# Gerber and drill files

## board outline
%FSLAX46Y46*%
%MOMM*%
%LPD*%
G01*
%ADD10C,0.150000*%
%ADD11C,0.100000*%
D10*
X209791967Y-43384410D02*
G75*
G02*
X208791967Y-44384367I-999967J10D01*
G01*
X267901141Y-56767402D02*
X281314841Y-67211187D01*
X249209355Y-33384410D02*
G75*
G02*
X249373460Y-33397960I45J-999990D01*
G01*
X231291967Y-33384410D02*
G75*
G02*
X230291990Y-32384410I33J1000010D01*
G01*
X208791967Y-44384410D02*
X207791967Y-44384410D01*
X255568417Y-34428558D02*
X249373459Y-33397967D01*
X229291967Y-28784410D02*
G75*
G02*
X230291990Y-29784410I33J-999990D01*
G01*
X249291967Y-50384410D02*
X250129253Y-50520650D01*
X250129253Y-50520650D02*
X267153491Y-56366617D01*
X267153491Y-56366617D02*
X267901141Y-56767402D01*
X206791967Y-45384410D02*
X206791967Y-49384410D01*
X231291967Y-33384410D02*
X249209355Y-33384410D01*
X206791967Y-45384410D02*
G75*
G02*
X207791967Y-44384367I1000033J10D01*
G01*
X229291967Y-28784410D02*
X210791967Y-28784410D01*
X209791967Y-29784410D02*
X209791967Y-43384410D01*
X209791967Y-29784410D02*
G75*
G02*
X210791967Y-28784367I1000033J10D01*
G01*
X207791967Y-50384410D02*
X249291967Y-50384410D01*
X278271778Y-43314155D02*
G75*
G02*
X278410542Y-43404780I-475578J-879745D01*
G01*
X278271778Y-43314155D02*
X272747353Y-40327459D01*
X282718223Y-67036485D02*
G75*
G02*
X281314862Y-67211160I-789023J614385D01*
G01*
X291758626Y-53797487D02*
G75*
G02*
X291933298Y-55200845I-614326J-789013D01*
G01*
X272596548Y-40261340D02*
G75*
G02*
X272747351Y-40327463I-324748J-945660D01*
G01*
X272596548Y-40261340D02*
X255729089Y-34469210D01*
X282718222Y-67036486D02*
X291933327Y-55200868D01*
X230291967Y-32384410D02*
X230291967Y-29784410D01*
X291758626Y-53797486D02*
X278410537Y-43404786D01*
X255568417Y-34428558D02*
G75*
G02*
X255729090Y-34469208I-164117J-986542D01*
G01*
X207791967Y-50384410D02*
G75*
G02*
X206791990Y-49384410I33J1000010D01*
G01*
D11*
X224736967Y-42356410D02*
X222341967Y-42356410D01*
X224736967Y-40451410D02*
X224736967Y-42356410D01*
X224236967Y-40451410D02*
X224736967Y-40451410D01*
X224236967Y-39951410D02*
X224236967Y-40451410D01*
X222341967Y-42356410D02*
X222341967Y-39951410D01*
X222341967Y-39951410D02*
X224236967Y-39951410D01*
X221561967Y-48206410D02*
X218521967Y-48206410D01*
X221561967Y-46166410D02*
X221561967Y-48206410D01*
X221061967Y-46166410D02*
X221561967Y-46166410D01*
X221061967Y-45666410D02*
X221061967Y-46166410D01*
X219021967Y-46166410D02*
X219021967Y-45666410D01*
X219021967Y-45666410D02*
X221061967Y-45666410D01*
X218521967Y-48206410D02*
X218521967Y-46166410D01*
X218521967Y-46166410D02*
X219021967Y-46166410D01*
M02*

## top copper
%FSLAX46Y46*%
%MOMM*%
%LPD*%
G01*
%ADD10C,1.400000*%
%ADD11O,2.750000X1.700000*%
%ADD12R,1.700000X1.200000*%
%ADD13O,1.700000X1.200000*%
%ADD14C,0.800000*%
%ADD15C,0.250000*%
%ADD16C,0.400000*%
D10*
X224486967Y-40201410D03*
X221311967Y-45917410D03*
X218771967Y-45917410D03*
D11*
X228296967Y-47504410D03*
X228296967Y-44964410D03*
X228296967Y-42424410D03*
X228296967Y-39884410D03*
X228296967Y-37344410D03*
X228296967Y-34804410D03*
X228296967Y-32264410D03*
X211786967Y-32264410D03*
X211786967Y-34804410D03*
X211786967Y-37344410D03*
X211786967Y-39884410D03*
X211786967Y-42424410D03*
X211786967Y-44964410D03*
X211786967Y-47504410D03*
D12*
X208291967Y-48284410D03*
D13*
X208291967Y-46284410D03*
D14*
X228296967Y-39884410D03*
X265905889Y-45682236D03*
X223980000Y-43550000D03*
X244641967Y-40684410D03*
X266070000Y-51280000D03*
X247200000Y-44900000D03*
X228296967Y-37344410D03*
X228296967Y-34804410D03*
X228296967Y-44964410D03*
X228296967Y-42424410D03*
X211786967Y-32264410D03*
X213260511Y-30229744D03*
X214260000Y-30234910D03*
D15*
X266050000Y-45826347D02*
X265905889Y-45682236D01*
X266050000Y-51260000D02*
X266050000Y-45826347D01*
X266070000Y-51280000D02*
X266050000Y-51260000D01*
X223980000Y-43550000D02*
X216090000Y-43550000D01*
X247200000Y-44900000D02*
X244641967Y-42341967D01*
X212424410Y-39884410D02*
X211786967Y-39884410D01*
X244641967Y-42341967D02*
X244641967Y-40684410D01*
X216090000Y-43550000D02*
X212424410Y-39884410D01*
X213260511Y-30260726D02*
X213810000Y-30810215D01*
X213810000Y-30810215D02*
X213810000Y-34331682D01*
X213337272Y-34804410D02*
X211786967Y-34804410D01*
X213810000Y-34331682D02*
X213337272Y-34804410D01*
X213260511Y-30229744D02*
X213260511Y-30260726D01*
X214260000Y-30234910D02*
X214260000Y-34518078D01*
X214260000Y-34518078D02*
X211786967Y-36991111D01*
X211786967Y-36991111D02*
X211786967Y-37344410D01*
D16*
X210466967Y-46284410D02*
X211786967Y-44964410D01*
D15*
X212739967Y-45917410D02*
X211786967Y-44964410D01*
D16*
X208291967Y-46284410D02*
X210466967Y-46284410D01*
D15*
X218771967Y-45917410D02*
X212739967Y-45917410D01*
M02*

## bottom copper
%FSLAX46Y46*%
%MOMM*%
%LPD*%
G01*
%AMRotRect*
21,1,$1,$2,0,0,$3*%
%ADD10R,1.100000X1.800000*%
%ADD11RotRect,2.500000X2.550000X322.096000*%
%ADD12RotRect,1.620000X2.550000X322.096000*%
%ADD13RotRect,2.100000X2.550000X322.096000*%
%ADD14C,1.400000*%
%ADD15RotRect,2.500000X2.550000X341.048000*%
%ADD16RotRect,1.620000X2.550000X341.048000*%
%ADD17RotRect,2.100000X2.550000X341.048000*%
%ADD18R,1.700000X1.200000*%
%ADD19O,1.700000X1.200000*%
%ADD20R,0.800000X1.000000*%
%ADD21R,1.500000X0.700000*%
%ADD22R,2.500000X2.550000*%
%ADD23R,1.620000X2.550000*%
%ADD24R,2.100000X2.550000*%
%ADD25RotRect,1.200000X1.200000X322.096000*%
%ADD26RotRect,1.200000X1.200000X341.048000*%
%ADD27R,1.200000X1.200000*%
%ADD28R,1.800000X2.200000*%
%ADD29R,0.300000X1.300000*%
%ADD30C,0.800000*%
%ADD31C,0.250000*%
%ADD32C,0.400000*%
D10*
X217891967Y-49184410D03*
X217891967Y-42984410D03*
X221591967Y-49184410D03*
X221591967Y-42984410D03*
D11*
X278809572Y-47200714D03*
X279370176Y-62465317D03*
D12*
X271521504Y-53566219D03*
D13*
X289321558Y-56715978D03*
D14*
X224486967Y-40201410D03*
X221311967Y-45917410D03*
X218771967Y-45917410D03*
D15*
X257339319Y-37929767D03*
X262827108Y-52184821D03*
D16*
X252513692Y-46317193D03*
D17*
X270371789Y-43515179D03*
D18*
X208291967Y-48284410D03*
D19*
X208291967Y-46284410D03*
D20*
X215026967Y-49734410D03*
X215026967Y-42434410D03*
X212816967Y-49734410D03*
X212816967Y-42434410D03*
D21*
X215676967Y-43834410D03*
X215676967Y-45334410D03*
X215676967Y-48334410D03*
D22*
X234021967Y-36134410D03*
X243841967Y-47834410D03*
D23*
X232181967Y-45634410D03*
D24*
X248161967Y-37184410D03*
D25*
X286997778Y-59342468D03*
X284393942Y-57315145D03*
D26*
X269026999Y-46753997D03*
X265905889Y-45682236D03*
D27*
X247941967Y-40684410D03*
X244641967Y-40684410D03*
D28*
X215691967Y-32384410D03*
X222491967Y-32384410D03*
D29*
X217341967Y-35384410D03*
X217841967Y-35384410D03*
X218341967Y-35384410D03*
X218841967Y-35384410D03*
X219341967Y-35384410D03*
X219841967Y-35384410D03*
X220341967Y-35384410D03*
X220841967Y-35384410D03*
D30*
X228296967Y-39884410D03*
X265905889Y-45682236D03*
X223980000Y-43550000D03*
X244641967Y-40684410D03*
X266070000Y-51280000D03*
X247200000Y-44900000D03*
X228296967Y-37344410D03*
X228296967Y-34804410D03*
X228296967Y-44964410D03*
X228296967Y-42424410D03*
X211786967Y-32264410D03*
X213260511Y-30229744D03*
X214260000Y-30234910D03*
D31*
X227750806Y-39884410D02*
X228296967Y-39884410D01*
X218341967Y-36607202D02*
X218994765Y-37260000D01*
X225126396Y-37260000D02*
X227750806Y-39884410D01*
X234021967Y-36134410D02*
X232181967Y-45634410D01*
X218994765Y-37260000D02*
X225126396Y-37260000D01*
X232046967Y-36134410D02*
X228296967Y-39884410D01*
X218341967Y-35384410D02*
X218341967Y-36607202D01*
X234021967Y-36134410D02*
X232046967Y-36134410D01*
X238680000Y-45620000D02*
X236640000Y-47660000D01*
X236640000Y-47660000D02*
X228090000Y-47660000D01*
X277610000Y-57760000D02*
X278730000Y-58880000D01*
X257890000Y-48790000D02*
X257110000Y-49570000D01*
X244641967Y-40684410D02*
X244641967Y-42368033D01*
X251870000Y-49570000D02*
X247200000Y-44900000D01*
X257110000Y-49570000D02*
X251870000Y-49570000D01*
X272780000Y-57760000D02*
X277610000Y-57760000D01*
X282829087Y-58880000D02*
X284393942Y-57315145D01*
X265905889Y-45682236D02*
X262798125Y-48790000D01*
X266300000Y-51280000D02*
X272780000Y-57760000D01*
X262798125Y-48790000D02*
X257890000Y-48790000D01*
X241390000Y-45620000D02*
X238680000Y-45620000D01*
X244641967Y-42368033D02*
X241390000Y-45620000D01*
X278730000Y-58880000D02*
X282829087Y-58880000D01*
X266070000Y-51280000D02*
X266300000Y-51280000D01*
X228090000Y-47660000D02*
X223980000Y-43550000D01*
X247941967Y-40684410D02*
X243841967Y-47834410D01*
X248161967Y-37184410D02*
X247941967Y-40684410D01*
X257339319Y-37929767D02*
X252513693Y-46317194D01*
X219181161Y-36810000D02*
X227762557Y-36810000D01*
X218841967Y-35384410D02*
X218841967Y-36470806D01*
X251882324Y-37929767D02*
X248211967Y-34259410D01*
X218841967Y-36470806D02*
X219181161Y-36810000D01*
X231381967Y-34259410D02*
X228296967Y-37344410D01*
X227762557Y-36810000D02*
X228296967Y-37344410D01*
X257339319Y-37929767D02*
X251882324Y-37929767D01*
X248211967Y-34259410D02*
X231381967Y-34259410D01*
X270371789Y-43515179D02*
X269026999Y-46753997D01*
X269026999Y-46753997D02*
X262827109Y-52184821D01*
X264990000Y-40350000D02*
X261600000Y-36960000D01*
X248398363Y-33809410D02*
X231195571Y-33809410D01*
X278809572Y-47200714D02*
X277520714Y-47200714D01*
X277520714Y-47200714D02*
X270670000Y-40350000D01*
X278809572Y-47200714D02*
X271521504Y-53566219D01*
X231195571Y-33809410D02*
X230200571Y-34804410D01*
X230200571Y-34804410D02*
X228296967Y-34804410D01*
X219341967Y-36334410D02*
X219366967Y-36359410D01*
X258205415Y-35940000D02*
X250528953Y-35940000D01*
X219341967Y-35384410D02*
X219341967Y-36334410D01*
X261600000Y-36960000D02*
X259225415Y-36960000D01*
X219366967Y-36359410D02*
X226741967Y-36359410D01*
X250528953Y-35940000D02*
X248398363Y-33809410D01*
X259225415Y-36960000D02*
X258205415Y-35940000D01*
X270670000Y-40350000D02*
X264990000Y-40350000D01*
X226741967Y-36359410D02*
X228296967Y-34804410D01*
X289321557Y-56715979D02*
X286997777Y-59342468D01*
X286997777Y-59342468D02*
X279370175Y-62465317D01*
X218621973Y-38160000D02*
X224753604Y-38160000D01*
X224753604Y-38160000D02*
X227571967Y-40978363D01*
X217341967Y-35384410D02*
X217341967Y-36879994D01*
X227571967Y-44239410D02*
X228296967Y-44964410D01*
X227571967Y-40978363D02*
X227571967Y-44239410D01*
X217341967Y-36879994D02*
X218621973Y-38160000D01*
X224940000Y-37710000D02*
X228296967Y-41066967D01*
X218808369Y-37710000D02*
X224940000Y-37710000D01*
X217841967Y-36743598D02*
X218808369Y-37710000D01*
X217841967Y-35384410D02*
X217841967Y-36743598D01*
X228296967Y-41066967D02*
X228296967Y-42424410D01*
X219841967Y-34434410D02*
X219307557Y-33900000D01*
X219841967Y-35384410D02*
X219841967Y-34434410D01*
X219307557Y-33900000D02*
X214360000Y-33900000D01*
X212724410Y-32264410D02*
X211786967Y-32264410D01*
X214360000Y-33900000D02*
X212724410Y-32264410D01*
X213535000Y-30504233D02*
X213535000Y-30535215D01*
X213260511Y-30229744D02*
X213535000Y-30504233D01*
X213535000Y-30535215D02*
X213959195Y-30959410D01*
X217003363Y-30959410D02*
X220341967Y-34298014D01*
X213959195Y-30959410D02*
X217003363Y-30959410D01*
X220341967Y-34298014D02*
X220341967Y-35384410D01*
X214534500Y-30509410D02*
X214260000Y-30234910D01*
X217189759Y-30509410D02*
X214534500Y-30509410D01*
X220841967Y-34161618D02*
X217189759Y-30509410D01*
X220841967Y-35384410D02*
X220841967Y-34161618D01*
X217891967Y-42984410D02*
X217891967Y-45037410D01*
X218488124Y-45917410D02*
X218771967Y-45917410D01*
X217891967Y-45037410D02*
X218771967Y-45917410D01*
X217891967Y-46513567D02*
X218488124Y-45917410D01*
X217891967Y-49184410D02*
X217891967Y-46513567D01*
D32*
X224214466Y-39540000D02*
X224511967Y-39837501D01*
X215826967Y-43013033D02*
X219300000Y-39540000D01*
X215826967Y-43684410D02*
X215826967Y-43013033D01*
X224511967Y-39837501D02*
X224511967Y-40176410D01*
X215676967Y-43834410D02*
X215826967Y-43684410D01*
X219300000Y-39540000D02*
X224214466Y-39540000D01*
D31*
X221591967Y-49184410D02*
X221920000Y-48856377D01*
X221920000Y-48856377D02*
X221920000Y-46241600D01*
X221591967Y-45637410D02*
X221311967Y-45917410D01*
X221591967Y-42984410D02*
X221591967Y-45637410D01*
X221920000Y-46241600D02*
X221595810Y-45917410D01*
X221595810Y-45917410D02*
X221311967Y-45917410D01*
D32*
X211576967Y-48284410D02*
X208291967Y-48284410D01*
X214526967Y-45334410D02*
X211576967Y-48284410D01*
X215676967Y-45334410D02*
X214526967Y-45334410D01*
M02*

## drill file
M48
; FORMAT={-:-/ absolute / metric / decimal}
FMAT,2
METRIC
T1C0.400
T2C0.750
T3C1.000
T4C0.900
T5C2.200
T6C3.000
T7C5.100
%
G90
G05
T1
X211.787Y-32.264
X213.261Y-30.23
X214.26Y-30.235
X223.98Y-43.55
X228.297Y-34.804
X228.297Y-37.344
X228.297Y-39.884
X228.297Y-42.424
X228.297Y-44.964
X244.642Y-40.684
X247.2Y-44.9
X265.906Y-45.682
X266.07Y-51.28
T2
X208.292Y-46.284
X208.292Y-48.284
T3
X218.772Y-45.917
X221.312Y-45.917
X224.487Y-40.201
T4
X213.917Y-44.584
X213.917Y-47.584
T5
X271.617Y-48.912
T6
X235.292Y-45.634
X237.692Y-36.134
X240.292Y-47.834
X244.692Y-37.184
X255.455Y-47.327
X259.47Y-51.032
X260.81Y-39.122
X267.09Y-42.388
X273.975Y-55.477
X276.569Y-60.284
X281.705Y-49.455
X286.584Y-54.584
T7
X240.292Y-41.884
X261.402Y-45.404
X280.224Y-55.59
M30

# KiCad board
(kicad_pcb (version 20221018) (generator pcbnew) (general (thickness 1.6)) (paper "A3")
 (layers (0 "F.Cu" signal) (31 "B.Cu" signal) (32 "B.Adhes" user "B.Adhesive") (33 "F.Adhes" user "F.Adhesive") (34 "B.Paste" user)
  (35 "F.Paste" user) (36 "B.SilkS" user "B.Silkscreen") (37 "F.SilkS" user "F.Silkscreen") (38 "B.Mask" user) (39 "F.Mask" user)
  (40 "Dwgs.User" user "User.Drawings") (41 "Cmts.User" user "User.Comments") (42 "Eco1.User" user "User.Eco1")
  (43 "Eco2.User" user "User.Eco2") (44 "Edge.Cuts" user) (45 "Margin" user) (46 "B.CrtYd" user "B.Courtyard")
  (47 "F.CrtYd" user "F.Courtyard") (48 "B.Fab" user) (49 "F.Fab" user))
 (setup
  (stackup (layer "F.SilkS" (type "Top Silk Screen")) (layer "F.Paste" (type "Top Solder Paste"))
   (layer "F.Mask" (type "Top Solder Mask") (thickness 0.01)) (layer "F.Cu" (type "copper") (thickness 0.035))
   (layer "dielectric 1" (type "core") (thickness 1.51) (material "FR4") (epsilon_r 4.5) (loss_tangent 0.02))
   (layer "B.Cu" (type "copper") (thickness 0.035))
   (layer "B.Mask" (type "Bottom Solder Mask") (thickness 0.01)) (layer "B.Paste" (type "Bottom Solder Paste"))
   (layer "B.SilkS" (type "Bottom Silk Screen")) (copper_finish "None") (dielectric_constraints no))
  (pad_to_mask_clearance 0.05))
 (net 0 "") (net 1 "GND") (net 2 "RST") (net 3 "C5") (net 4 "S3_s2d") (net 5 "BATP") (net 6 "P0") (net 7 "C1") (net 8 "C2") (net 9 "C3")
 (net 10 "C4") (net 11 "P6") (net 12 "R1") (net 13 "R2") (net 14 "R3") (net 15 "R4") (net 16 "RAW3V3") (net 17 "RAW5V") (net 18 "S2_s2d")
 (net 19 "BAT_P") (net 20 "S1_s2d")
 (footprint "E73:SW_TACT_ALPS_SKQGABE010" (layer "F.Cu") (at 219.741967 46.08441 90)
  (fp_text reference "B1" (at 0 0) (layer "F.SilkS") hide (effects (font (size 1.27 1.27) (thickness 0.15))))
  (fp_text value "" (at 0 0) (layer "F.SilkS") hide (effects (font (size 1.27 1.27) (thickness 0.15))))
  (pad "1" smd rect (at -3.1 -1.85 90) (size 1.8 1.1) (layers "B.Cu" "B.Paste" "B.Mask") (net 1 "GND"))
  (pad "1" smd rect (at 3.1 -1.85 90) (size 1.8 1.1) (layers "B.Cu" "B.Paste" "B.Mask") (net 1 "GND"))
  (pad "2" smd rect (at -3.1 1.85 90) (size 1.8 1.1) (layers "B.Cu" "B.Paste" "B.Mask") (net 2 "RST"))
  (pad "2" smd rect (at 3.1 1.85 90) (size 1.8 1.1) (layers "B.Cu" "B.Paste" "B.Mask") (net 2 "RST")))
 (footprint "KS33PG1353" (layer "F.Cu") (at 280.224404 55.589614 -37.904)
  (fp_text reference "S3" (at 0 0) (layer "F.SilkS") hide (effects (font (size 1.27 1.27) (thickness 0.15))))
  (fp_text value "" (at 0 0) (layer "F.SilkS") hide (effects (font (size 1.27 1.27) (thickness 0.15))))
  (pad "" np_thru_hole circle (at -5 3.75) (size 3 3) (drill 3) (layers "*.Cu" "*.Mask"))
  (pad "" np_thru_hole circle (at -2.6 -5.75) (size 3 3) (drill 3) (layers "*.Cu" "*.Mask"))
  (pad "" np_thru_hole circle (at 0 0) (size 5.1 5.1) (drill 5.1) (layers "*.Cu" "*.Mask"))
  (pad "" np_thru_hole circle (at 0 5.95) (size 3 3) (drill 3) (layers "*.Cu" "*.Mask"))
  (pad "" np_thru_hole circle (at 4.4 -4.7) (size 3 3) (drill 3) (layers "*.Cu" "*.Mask"))
  (pad "1" smd rect (at -6.27 -5.75 322.096) (size 2.5 2.55) (layers "B.Cu" "B.Paste" "B.Mask") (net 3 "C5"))
  (pad "1" smd rect (at 3.55 5.95 322.096) (size 2.5 2.55) (layers "B.Cu" "B.Paste" "B.Mask") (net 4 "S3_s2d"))
  (pad "2" smd rect (at -8.11 3.75 322.096) (size 1.62 2.55) (layers "B.Cu" "B.Paste" "B.Mask") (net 3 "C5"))
  (pad "2" smd rect (at 7.87 -4.7 322.096) (size 2.1 2.55) (layers "B.Cu" "B.Paste" "B.Mask") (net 4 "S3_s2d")))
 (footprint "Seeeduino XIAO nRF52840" (layer "F.Cu") (at 220.041967 39.88441 180)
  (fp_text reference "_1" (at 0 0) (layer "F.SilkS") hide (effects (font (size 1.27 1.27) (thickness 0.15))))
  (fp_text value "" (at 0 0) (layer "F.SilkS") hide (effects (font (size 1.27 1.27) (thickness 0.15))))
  (fp_line (start -4.695 -2.472) (end -2.3 -2.472) (stroke (width 0.1) (type solid)) (layer "Edge.Cuts"))
  (fp_line (start -4.695 -0.567) (end -4.695 -2.472) (stroke (width 0.1) (type solid)) (layer "Edge.Cuts"))
  (fp_line (start -4.195 -0.567) (end -4.695 -0.567) (stroke (width 0.1) (type solid)) (layer "Edge.Cuts"))
  (fp_line (start -4.195 -0.067) (end -4.195 -0.567) (stroke (width 0.1) (type solid)) (layer "Edge.Cuts"))
  (fp_line (start -2.3 -2.472) (end -2.3 -0.067) (stroke (width 0.1) (type solid)) (layer "Edge.Cuts"))
  (fp_line (start -2.3 -0.067) (end -4.195 -0.067) (stroke (width 0.1) (type solid)) (layer "Edge.Cuts"))
  (fp_line (start -1.52 -8.322) (end 1.52 -8.322) (stroke (width 0.1) (type solid)) (layer "Edge.Cuts"))
  (fp_line (start -1.52 -6.282) (end -1.52 -8.322) (stroke (width 0.1) (type solid)) (layer "Edge.Cuts"))
  (fp_line (start -1.02 -6.282) (end -1.52 -6.282) (stroke (width 0.1) (type solid)) (layer "Edge.Cuts"))
  (fp_line (start -1.02 -5.782) (end -1.02 -6.282) (stroke (width 0.1) (type solid)) (layer "Edge.Cuts"))
  (fp_line (start 1.02 -6.282) (end 1.02 -5.782) (stroke (width 0.1) (type solid)) (layer "Edge.Cuts"))
  (fp_line (start 1.02 -5.782) (end -1.02 -5.782) (stroke (width 0.1) (type solid)) (layer "Edge.Cuts"))
  (fp_line (start 1.52 -8.322) (end 1.52 -6.282) (stroke (width 0.1) (type solid)) (layer "Edge.Cuts"))
  (fp_line (start 1.52 -6.282) (end 1.02 -6.282) (stroke (width 0.1) (type solid)) (layer "Edge.Cuts"))
  (pad "" thru_hole circle (at -4.445 -0.317) (size 1.4 1.4) (drill 1) (layers "*.Cu" "*.Mask") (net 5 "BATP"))
  (pad "" thru_hole circle (at -1.27 -6.033) (size 1.4 1.4) (drill 1) (layers "*.Cu" "*.Mask") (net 2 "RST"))
  (pad "" thru_hole circle (at 1.27 -6.033) (size 1.4 1.4) (drill 1) (layers "*.Cu" "*.Mask") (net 1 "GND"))
  (pad "1" smd oval (at -8.255 -7.62 180) (size 2.75 1.7) (layers "F.Cu" "F.Paste" "F.Mask") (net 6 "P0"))
  (pad "2" smd oval (at -8.255 -5.08 180) (size 2.75 1.7) (layers "F.Cu" "F.Paste" "F.Mask") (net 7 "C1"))
  (pad "3" smd oval (at -8.255 -2.54 180) (size 2.75 1.7) (layers "F.Cu" "F.Paste" "F.Mask") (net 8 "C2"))
  (pad "4" smd oval (at -8.255 0 180) (size 2.75 1.7) (layers "F.Cu" "F.Paste" "F.Mask") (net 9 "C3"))
  (pad "5" smd oval (at -8.255 2.54 180) (size 2.75 1.7) (layers "F.Cu" "F.Paste" "F.Mask") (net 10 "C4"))
  (pad "6" smd oval (at -8.255 5.08 180) (size 2.75 1.7) (layers "F.Cu" "F.Paste" "F.Mask") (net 3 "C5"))
  (pad "7" smd oval (at -8.255 7.62 180) (size 2.75 1.7) (layers "F.Cu" "F.Paste" "F.Mask") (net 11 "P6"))
  (pad "8" smd oval (at 8.255 7.62 180) (size 2.75 1.7) (layers "F.Cu" "F.Paste" "F.Mask") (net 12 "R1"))
  (pad "9" smd oval (at 8.255 5.08 180) (size 2.75 1.7) (layers "F.Cu" "F.Paste" "F.Mask") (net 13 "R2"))
  (pad "10" smd oval (at 8.255 2.54 180) (size 2.75 1.7) (layers "F.Cu" "F.Paste" "F.Mask") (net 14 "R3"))
  (pad "11" smd oval (at 8.255 0 180) (size 2.75 1.7) (layers "F.Cu" "F.Paste" "F.Mask") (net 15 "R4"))
  (pad "12" smd oval (at 8.255 -2.54 180) (size 2.75 1.7) (layers "F.Cu" "F.Paste" "F.Mask") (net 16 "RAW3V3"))
  (pad "13" smd oval (at 8.255 -5.08 180) (size 2.75 1.7) (layers "F.Cu" "F.Paste" "F.Mask") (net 1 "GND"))
  (pad "14" smd oval (at 8.255 -7.62 180) (size 2.75 1.7) (layers "F.Cu" "F.Paste" "F.Mask") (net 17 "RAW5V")))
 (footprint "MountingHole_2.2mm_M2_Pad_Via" (layer "F.Cu") (at 271.61651 48.91199 -18.952)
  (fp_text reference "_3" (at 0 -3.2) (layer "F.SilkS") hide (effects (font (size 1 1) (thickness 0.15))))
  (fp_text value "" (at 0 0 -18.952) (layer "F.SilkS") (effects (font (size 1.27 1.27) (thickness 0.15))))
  (pad "" np_thru_hole circle (at 0 0) (size 2.2 2.2) (drill 2.2) (layers "*.Cu" "*.Mask")))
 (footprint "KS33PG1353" (layer "F.Cu") (at 261.401967 45.40441 -18.952)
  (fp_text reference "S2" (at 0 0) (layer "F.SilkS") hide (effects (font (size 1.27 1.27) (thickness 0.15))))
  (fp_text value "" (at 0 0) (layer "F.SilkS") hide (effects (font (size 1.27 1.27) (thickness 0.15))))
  (pad "" np_thru_hole circle (at -5 3.75) (size 3 3) (drill 3) (layers "*.Cu" "*.Mask"))
  (pad "" np_thru_hole circle (at -2.6 -5.75) (size 3 3) (drill 3) (layers "*.Cu" "*.Mask"))
  (pad "" np_thru_hole circle (at 0 0) (size 5.1 5.1) (drill 5.1) (layers "*.Cu" "*.Mask"))
  (pad "" np_thru_hole circle (at 0 5.95) (size 3 3) (drill 3) (layers "*.Cu" "*.Mask"))
  (pad "" np_thru_hole circle (at 4.4 -4.7) (size 3 3) (drill 3) (layers "*.Cu" "*.Mask"))
  (pad "1" smd rect (at -6.27 -5.75 341.048) (size 2.5 2.55) (layers "B.Cu" "B.Paste" "B.Mask") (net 10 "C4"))
  (pad "1" smd rect (at 3.55 5.95 341.048) (size 2.5 2.55) (layers "B.Cu" "B.Paste" "B.Mask") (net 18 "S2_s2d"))
  (pad "2" smd rect (at -8.11 3.75 341.048) (size 1.62 2.55) (layers "B.Cu" "B.Paste" "B.Mask") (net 10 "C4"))
  (pad "2" smd rect (at 7.87 -4.7 341.048) (size 2.1 2.55) (layers "B.Cu" "B.Paste" "B.Mask") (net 18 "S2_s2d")))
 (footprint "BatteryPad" (layer "F.Cu") (at 208.291967 47.28441 90)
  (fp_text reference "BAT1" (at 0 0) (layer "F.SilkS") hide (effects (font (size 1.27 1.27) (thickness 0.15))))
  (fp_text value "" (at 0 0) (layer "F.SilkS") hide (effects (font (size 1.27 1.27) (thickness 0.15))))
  (pad "1" thru_hole rect (at -1 0 90) (size 1.2 1.7) (drill 0.75) (layers "*.Cu" "*.Mask") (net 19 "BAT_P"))
  (pad "2" thru_hole oval (at 1 0 90) (size 1.2 1.7) (drill 0.75) (layers "*.Cu" "*.Mask") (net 1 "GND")))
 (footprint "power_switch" (layer "F.Cu") (at 213.941967 46.08441 180)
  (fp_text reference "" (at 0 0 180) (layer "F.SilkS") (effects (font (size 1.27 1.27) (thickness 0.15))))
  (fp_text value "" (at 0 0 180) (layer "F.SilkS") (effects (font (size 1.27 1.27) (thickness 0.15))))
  (pad "" smd rect (at -1.085 -3.65 90) (size 1 0.8) (layers "B.Cu" "B.Paste" "B.Mask"))
  (pad "" smd rect (at -1.085 3.65 90) (size 1 0.8) (layers "B.Cu" "B.Paste" "B.Mask"))
  (pad "" np_thru_hole circle (at 0.025 -1.5 270) (size 0.9 0.9) (drill 0.9) (layers "*.Cu" "*.Mask"))
  (pad "" np_thru_hole circle (at 0.025 1.5 270) (size 0.9 0.9) (drill 0.9) (layers "*.Cu" "*.Mask"))
  (pad "" smd rect (at 1.125 -3.65 90) (size 1 0.8) (layers "B.Cu" "B.Paste" "B.Mask"))
  (pad "" smd rect (at 1.125 3.65 90) (size 1 0.8) (layers "B.Cu" "B.Paste" "B.Mask"))
  (pad "4" smd rect (at -1.735 2.25 90) (size 0.7 1.5) (layers "B.Cu" "B.Paste" "B.Mask") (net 5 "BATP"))
  (pad "5" smd rect (at -1.735 0.75 90) (size 0.7 1.5) (layers "B.Cu" "B.Paste" "B.Mask") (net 19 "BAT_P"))
  (pad "6" smd rect (at -1.735 -2.25 90) (size 0.7 1.5) (layers "B.Cu" "B.Paste" "B.Mask")))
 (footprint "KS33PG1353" (layer "F.Cu") (at 240.291967 41.88441)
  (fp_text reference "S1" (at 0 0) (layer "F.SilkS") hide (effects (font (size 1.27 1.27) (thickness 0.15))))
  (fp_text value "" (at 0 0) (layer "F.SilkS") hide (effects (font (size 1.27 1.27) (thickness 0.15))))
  (pad "" np_thru_hole circle (at -5 3.75) (size 3 3) (drill 3) (layers "*.Cu" "*.Mask"))
  (pad "" np_thru_hole circle (at -2.6 -5.75) (size 3 3) (drill 3) (layers "*.Cu" "*.Mask"))
  (pad "" np_thru_hole circle (at 0 0) (size 5.1 5.1) (drill 5.1) (layers "*.Cu" "*.Mask"))
  (pad "" np_thru_hole circle (at 0 5.95) (size 3 3) (drill 3) (layers "*.Cu" "*.Mask"))
  (pad "" np_thru_hole circle (at 4.4 -4.7) (size 3 3) (drill 3) (layers "*.Cu" "*.Mask"))
  (pad "1" smd rect (at -6.27 -5.75) (size 2.5 2.55) (layers "B.Cu" "B.Paste" "B.Mask") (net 9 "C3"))
  (pad "1" smd rect (at 3.55 5.95) (size 2.5 2.55) (layers "B.Cu" "B.Paste" "B.Mask") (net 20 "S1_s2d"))
  (pad "2" smd rect (at -8.11 3.75) (size 1.62 2.55) (layers "B.Cu" "B.Paste" "B.Mask") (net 9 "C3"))
  (pad "2" smd rect (at 7.87 -4.7) (size 2.1 2.55) (layers "B.Cu" "B.Paste" "B.Mask") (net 20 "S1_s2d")))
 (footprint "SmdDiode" (layer "B.Cu") (at 280.224404 55.589614 -37.904)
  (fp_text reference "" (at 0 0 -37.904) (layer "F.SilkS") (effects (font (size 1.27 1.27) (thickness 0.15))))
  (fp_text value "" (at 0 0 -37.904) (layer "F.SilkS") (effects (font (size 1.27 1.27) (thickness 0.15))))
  (pad "1" smd rect (at 7.65 -1.2 322.096) (size 1.2 1.2) (layers "B.Cu" "B.Paste" "B.Mask") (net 4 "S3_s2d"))
  (pad "2" smd rect (at 4.35 -1.2 322.096) (size 1.2 1.2) (layers "B.Cu" "B.Paste" "B.Mask") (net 15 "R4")))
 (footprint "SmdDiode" (layer "B.Cu") (at 261.401967 45.40441 -18.952)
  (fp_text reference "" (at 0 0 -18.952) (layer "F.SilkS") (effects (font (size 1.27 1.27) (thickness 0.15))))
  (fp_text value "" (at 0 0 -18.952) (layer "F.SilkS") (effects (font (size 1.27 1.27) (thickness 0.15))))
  (pad "1" smd rect (at 7.65 -1.2 341.048) (size 1.2 1.2) (layers "B.Cu" "B.Paste" "B.Mask") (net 18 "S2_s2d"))
  (pad "2" smd rect (at 4.35 -1.2 341.048) (size 1.2 1.2) (layers "B.Cu" "B.Paste" "B.Mask") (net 15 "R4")))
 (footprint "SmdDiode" (layer "B.Cu") (at 240.291967 41.88441)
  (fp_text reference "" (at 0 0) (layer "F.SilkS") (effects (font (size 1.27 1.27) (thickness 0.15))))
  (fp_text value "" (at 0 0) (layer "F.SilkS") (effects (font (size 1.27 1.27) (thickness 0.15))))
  (pad "1" smd rect (at 7.65 -1.2) (size 1.2 1.2) (layers "B.Cu" "B.Paste" "B.Mask") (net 20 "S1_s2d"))
  (pad "2" smd rect (at 4.35 -1.2) (size 1.2 1.2) (layers "B.Cu" "B.Paste" "B.Mask") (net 15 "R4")))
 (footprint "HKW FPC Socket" (layer "B.Cu") (at 219.091967 32.38441)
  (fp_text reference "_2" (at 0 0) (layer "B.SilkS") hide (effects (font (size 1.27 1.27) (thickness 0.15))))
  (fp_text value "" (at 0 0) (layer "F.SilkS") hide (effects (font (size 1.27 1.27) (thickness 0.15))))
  (pad "" smd rect (at -3.4 0) (size 1.8 2.2) (layers "B.Cu" "B.Paste" "B.Mask"))
  (pad "" smd rect (at 3.4 0) (size 1.8 2.2) (layers "B.Cu" "B.Paste" "B.Mask"))
  (pad "1" smd rect (at -1.75 3) (size 0.3 1.3) (layers "B.Cu" "B.Paste" "B.Mask") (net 7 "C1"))
  (pad "2" smd rect (at -1.25 3) (size 0.3 1.3) (layers "B.Cu" "B.Paste" "B.Mask") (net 8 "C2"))
  (pad "3" smd rect (at -0.75 3) (size 0.3 1.3) (layers "B.Cu" "B.Paste" "B.Mask") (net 9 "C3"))
  (pad "4" smd rect (at -0.25 3) (size 0.3 1.3) (layers "B.Cu" "B.Paste" "B.Mask") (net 10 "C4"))
  (pad "5" smd rect (at 0.25 3) (size 0.3 1.3) (layers "B.Cu" "B.Paste" "B.Mask") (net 3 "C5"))
  (pad "6" smd rect (at 0.75 3) (size 0.3 1.3) (layers "B.Cu" "B.Paste" "B.Mask") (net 12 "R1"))
  (pad "7" smd rect (at 1.25 3) (size 0.3 1.3) (layers "B.Cu" "B.Paste" "B.Mask") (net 13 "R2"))
  (pad "8" smd rect (at 1.75 3) (size 0.3 1.3) (layers "B.Cu" "B.Paste" "B.Mask") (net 14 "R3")))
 (gr_arc (start 209.791967 43.38441) (mid 209.499074 44.091517) (end 208.791967 44.38441) (stroke (width 0.15) (type solid))
  (layer "Edge.Cuts"))
 (gr_line (start 267.901141 56.767402) (end 281.314841 67.211187) (stroke (width 0.15) (type solid)) (layer "Edge.Cuts"))
 (gr_arc (start 249.209355 33.38441) (mid 249.291687 33.387805) (end 249.373459 33.397967) (stroke (width 0.15) (type solid))
  (layer "Edge.Cuts"))
 (gr_arc (start 231.291967 33.38441) (mid 230.58486 33.091517) (end 230.291967 32.38441) (stroke (width 0.15) (type solid))
  (layer "Edge.Cuts"))
 (gr_line (start 208.791967 44.38441) (end 207.791967 44.38441) (stroke (width 0.15) (type solid)) (layer "Edge.Cuts"))
 (gr_line (start 255.568417 34.428558) (end 249.373459 33.397967) (stroke (width 0.15) (type solid)) (layer "Edge.Cuts"))
 (gr_arc (start 229.291967 28.78441) (mid 229.999074 29.077303) (end 230.291967 29.78441) (stroke (width 0.15) (type solid))
  (layer "Edge.Cuts"))
 (gr_line (start 249.291967 50.38441) (end 250.129253 50.52065) (stroke (width 0.15) (type solid)) (layer "Edge.Cuts"))
 (gr_line (start 250.129253 50.52065) (end 267.153491 56.366617) (stroke (width 0.15) (type solid)) (layer "Edge.Cuts"))
 (gr_line (start 267.153491 56.366617) (end 267.901141 56.767402) (stroke (width 0.15) (type solid)) (layer "Edge.Cuts"))
 (gr_line (start 206.791967 45.38441) (end 206.791967 49.38441) (stroke (width 0.15) (type solid)) (layer "Edge.Cuts"))
 (gr_line (start 231.291967 33.38441) (end 249.209355 33.38441) (stroke (width 0.15) (type solid)) (layer "Edge.Cuts"))
 (gr_arc (start 206.791967 45.38441) (mid 207.08486 44.677303) (end 207.791967 44.38441) (stroke (width 0.15) (type solid))
  (layer "Edge.Cuts"))
 (gr_line (start 229.291967 28.78441) (end 210.791967 28.78441) (stroke (width 0.15) (type solid)) (layer "Edge.Cuts"))
 (gr_line (start 209.791967 29.78441) (end 209.791967 43.38441) (stroke (width 0.15) (type solid)) (layer "Edge.Cuts"))
 (gr_arc (start 209.791967 29.78441) (mid 210.08486 29.077303) (end 210.791967 28.78441) (stroke (width 0.15) (type solid))
  (layer "Edge.Cuts"))
 (gr_line (start 207.791967 50.38441) (end 249.291967 50.38441) (stroke (width 0.15) (type solid)) (layer "Edge.Cuts"))
 (gr_arc (start 278.271778 43.314155) (mid 278.343038 43.356591) (end 278.410537 43.404786) (stroke (width 0.15) (type solid))
  (layer "Edge.Cuts"))
 (gr_line (start 278.271778 43.314155) (end 272.747353 40.327459) (stroke (width 0.15) (type solid)) (layer "Edge.Cuts"))
 (gr_arc (start 282.718223 67.036485) (mid 282.052714 67.414486) (end 281.314841 67.211187) (stroke (width 0.15) (type solid))
  (layer "Edge.Cuts"))
 (gr_arc (start 291.758626 53.797487) (mid 292.136626 54.462996) (end 291.933327 55.200868) (stroke (width 0.15) (type solid))
  (layer "Edge.Cuts"))
 (gr_arc (start 272.596548 40.26134) (mid 272.673314 40.29129) (end 272.747353 40.327459) (stroke (width 0.15) (type solid))
  (layer "Edge.Cuts"))
 (gr_line (start 272.596548 40.26134) (end 255.729089 34.46921) (stroke (width 0.15) (type solid)) (layer "Edge.Cuts"))
 (gr_line (start 282.718222 67.036486) (end 291.933327 55.200868) (stroke (width 0.15) (type solid)) (layer "Edge.Cuts"))
 (gr_line (start 230.291967 32.38441) (end 230.291967 29.78441) (stroke (width 0.15) (type solid)) (layer "Edge.Cuts"))
 (gr_line (start 291.758626 53.797486) (end 278.410537 43.404786) (stroke (width 0.15) (type solid)) (layer "Edge.Cuts"))
 (gr_arc (start 255.568417 34.428558) (mid 255.649597 34.44555) (end 255.729089 34.46921) (stroke (width 0.15) (type solid))
  (layer "Edge.Cuts"))
 (gr_arc (start 207.791967 50.38441) (mid 207.08486 50.091517) (end 206.791967 49.38441) (stroke (width 0.15) (type solid))
  (layer "Edge.Cuts"))
 (via (at 228.296967 39.88441) (size 0.8) (drill 0.4) (layers "F.Cu" "B.Cu") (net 9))
 (segment (start 227.750806 39.88441) (end 228.296967 39.88441) (width 0.25) (layer "B.Cu") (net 9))
 (segment (start 218.341967 36.607202) (end 218.994765 37.26) (width 0.25) (layer "B.Cu") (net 9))
 (segment (start 225.126396 37.26) (end 227.750806 39.88441) (width 0.25) (layer "B.Cu") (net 9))
 (segment (start 234.021967 36.13441) (end 232.181967 45.63441) (width 0.25) (layer "B.Cu") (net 9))
 (segment (start 218.994765 37.26) (end 225.126396 37.26) (width 0.25) (layer "B.Cu") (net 9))
 (segment (start 232.046967 36.13441) (end 228.296967 39.88441) (width 0.25) (layer "B.Cu") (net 9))
 (segment (start 218.341967 35.38441) (end 218.341967 36.607202) (width 0.25) (layer "B.Cu") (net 9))
 (segment (start 234.021967 36.13441) (end 232.046967 36.13441) (width 0.25) (layer "B.Cu") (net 9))
 (segment (start 266.05 45.826347) (end 265.905889 45.682236) (width 0.25) (layer "F.Cu") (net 15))
 (segment (start 266.05 51.26) (end 266.05 45.826347) (width 0.25) (layer "F.Cu") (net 15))
 (segment (start 266.07 51.28) (end 266.05 51.26) (width 0.25) (layer "F.Cu") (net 15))
 (segment (start 223.98 43.55) (end 216.09 43.55) (width 0.25) (layer "F.Cu") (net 15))
 (segment (start 247.2 44.9) (end 244.641967 42.341967) (width 0.25) (layer "F.Cu") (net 15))
 (segment (start 212.42441 39.88441) (end 211.786967 39.88441) (width 0.25) (layer "F.Cu") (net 15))
 (segment (start 244.641967 42.341967) (end 244.641967 40.68441) (width 0.25) (layer "F.Cu") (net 15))
 (segment (start 216.09 43.55) (end 212.42441 39.88441) (width 0.25) (layer "F.Cu") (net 15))
 (via (at 265.905889 45.682236) (size 0.8) (drill 0.4) (layers "F.Cu" "B.Cu") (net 15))
 (via (at 223.98 43.55) (size 0.8) (drill 0.4) (layers "F.Cu" "B.Cu") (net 15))
 (via (at 244.641967 40.68441) (size 0.8) (drill 0.4) (layers "F.Cu" "B.Cu") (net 15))
 (via (at 266.07 51.28) (size 0.8) (drill 0.4) (layers "F.Cu" "B.Cu") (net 15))
 (via (at 247.2 44.9) (size 0.8) (drill 0.4) (layers "F.Cu" "B.Cu") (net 15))
 (segment (start 238.68 45.62) (end 236.64 47.66) (width 0.25) (layer "B.Cu") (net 15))
 (segment (start 236.64 47.66) (end 228.09 47.66) (width 0.25) (layer "B.Cu") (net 15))
 (segment (start 277.61 57.76) (end 278.73 58.88) (width 0.25) (layer "B.Cu") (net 15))
 (segment (start 257.89 48.79) (end 257.11 49.57) (width 0.25) (layer "B.Cu") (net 15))
 (segment (start 244.641967 40.68441) (end 244.641967 42.368033) (width 0.25) (layer "B.Cu") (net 15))
 (segment (start 251.87 49.57) (end 247.2 44.9) (width 0.25) (layer "B.Cu") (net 15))
 (segment (start 257.11 49.57) (end 251.87 49.57) (width 0.25) (layer "B.Cu") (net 15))
 (segment (start 272.78 57.76) (end 277.61 57.76) (width 0.25) (layer "B.Cu") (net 15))
 (segment (start 282.829087 58.88) (end 284.393942 57.315145) (width 0.25) (layer "B.Cu") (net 15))
 (segment (start 265.905889 45.682236) (end 262.798125 48.79) (width 0.25) (layer "B.Cu") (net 15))
 (segment (start 266.3 51.28) (end 272.78 57.76) (width 0.25) (layer "B.Cu") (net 15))
 (segment (start 262.798125 48.79) (end 257.89 48.79) (width 0.25) (layer "B.Cu") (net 15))
 (segment (start 241.39 45.62) (end 238.68 45.62) (width 0.25) (layer "B.Cu") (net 15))
 (segment (start 244.641967 42.368033) (end 241.39 45.62) (width 0.25) (layer "B.Cu") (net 15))
 (segment (start 278.73 58.88) (end 282.829087 58.88) (width 0.25) (layer "B.Cu") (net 15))
 (segment (start 266.07 51.28) (end 266.3 51.28) (width 0.25) (layer "B.Cu") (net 15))
 (segment (start 228.09 47.66) (end 223.98 43.55) (width 0.25) (layer "B.Cu") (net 15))
 (segment (start 247.941967 40.68441) (end 243.841967 47.83441) (width 0.25) (layer "B.Cu") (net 20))
 (segment (start 248.161967 37.18441) (end 247.941967 40.68441) (width 0.25) (layer "B.Cu") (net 20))
 (via (at 228.296967 37.34441) (size 0.8) (drill 0.4) (layers "F.Cu" "B.Cu") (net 10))
 (segment (start 257.339319 37.929767) (end 252.513693 46.317194) (width 0.25) (layer "B.Cu") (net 10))
 (segment (start 219.181161 36.81) (end 227.762557 36.81) (width 0.25) (layer "B.Cu") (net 10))
 (segment (start 218.841967 35.38441) (end 218.841967 36.470806) (width 0.25) (layer "B.Cu") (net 10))
 (segment (start 251.882324 37.929767) (end 248.211967 34.25941) (width 0.25) (layer "B.Cu") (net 10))
 (segment (start 218.841967 36.470806) (end 219.181161 36.81) (width 0.25) (layer "B.Cu") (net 10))
 (segment (start 231.381967 34.25941) (end 228.296967 37.34441) (width 0.25) (layer "B.Cu") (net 10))
 (segment (start 227.762557 36.81) (end 228.296967 37.34441) (width 0.25) (layer "B.Cu") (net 10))
 (segment (start 257.339319 37.929767) (end 251.882324 37.929767) (width 0.25) (layer "B.Cu") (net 10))
 (segment (start 248.211967 34.25941) (end 231.381967 34.25941) (width 0.25) (layer "B.Cu") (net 10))
 (segment (start 270.371789 43.515179) (end 269.026999 46.753997) (width 0.25) (layer "B.Cu") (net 18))
 (segment (start 269.026999 46.753997) (end 262.827109 52.184821) (width 0.25) (layer "B.Cu") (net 18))
 (via (at 228.296967 34.80441) (size 0.8) (drill 0.4) (layers "F.Cu" "B.Cu") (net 3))
 (segment (start 264.99 40.35) (end 261.6 36.96) (width 0.25) (layer "B.Cu") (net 3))
 (segment (start 248.398363 33.80941) (end 231.195571 33.80941) (width 0.25) (layer "B.Cu") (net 3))
 (segment (start 278.809572 47.200714) (end 277.520714 47.200714) (width 0.25) (layer "B.Cu") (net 3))
 (segment (start 277.520714 47.200714) (end 270.67 40.35) (width 0.25) (layer "B.Cu") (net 3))
 (segment (start 278.809572 47.200714) (end 271.521504 53.566219) (width 0.25) (layer "B.Cu") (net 3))
 (segment (start 231.195571 33.80941) (end 230.200571 34.80441) (width 0.25) (layer "B.Cu") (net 3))
 (segment (start 230.200571 34.80441) (end 228.296967 34.80441) (width 0.25) (layer "B.Cu") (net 3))
 (segment (start 219.341967 36.33441) (end 219.366967 36.35941) (width 0.25) (layer "B.Cu") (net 3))
 (segment (start 258.205415 35.94) (end 250.528953 35.94) (width 0.25) (layer "B.Cu") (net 3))
 (segment (start 219.341967 35.38441) (end 219.341967 36.33441) (width 0.25) (layer "B.Cu") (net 3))
 (segment (start 261.6 36.96) (end 259.225415 36.96) (width 0.25) (layer "B.Cu") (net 3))
 (segment (start 219.366967 36.35941) (end 226.741967 36.35941) (width 0.25) (layer "B.Cu") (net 3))
 (segment (start 250.528953 35.94) (end 248.398363 33.80941) (width 0.25) (layer "B.Cu") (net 3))
 (segment (start 259.225415 36.96) (end 258.205415 35.94) (width 0.25) (layer "B.Cu") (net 3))
 (segment (start 270.67 40.35) (end 264.99 40.35) (width 0.25) (layer "B.Cu") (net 3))
 (segment (start 226.741967 36.35941) (end 228.296967 34.80441) (width 0.25) (layer "B.Cu") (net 3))
 (segment (start 289.321557 56.715979) (end 286.997777 59.342468) (width 0.25) (layer "B.Cu") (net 4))
 (segment (start 286.997777 59.342468) (end 279.370175 62.465317) (width 0.25) (layer "B.Cu") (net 4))
 (via (at 228.296967 44.96441) (size 0.8) (drill 0.4) (layers "F.Cu" "B.Cu") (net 7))
 (segment (start 218.621973 38.16) (end 224.753604 38.16) (width 0.25) (layer "B.Cu") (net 7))
 (segment (start 224.753604 38.16) (end 227.571967 40.978363) (width 0.25) (layer "B.Cu") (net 7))
 (segment (start 217.341967 35.38441) (end 217.341967 36.879994) (width 0.25) (layer "B.Cu") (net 7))
 (segment (start 227.571967 44.23941) (end 228.296967 44.96441) (width 0.25) (layer "B.Cu") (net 7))
 (segment (start 227.571967 40.978363) (end 227.571967 44.23941) (width 0.25) (layer "B.Cu") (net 7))
 (segment (start 217.341967 36.879994) (end 218.621973 38.16) (width 0.25) (layer "B.Cu") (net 7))
 (via (at 228.296967 42.42441) (size 0.8) (drill 0.4) (layers "F.Cu" "B.Cu") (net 8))
 (segment (start 224.94 37.71) (end 228.296967 41.066967) (width 0.25) (layer "B.Cu") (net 8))
 (segment (start 218.808369 37.71) (end 224.94 37.71) (width 0.25) (layer "B.Cu") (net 8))
 (segment (start 217.841967 36.743598) (end 218.808369 37.71) (width 0.25) (layer "B.Cu") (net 8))
 (segment (start 217.841967 35.38441) (end 217.841967 36.743598) (width 0.25) (layer "B.Cu") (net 8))
 (segment (start 228.296967 41.066967) (end 228.296967 42.42441) (width 0.25) (layer "B.Cu") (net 8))
 (via (at 211.786967 32.26441) (size 0.8) (drill 0.4) (layers "F.Cu" "B.Cu") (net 12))
 (segment (start 219.841967 34.43441) (end 219.307557 33.9) (width 0.25) (layer "B.Cu") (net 12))
 (segment (start 219.841967 35.38441) (end 219.841967 34.43441) (width 0.25) (layer "B.Cu") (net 12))
 (segment (start 219.307557 33.9) (end 214.36 33.9) (width 0.25) (layer "B.Cu") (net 12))
 (segment (start 212.72441 32.26441) (end 211.786967 32.26441) (width 0.25) (layer "B.Cu") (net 12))
 (segment (start 214.36 33.9) (end 212.72441 32.26441) (width 0.25) (layer "B.Cu") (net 12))
 (segment (start 213.260511 30.260726) (end 213.81 30.810215) (width 0.25) (layer "F.Cu") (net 13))
 (segment (start 213.81 30.810215) (end 213.81 34.331682) (width 0.25) (layer "F.Cu") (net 13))
 (segment (start 213.337272 34.80441) (end 211.786967 34.80441) (width 0.25) (layer "F.Cu") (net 13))
 (segment (start 213.81 34.331682) (end 213.337272 34.80441) (width 0.25) (layer "F.Cu") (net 13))
 (segment (start 213.260511 30.229744) (end 213.260511 30.260726) (width 0.25) (layer "F.Cu") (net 13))
 (via (at 213.260511 30.229744) (size 0.8) (drill 0.4) (layers "F.Cu" "B.Cu") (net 13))
 (segment (start 213.535 30.504233) (end 213.535 30.535215) (width 0.25) (layer "B.Cu") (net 13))
 (segment (start 213.260511 30.229744) (end 213.535 30.504233) (width 0.25) (layer "B.Cu") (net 13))
 (segment (start 213.535 30.535215) (end 213.959195 30.95941) (width 0.25) (layer "B.Cu") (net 13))
 (segment (start 217.003363 30.95941) (end 220.341967 34.298014) (width 0.25) (layer "B.Cu") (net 13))
 (segment (start 213.959195 30.95941) (end 217.003363 30.95941) (width 0.25) (layer "B.Cu") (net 13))
 (segment (start 220.341967 34.298014) (end 220.341967 35.38441) (width 0.25) (layer "B.Cu") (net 13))
 (segment (start 214.26 30.23491) (end 214.26 34.518078) (width 0.25) (layer "F.Cu") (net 14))
 (segment (start 214.26 34.518078) (end 211.786967 36.991111) (width 0.25) (layer "F.Cu") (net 14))
 (segment (start 211.786967 36.991111) (end 211.786967 37.34441) (width 0.25) (layer "F.Cu") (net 14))
 (via (at 214.26 30.23491) (size 0.8) (drill 0.4) (layers "F.Cu" "B.Cu") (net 14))
 (segment (start 214.5345 30.50941) (end 214.26 30.23491) (width 0.25) (layer "B.Cu") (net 14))
 (segment (start 217.189759 30.50941) (end 214.5345 30.50941) (width 0.25) (layer "B.Cu") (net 14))
 (segment (start 220.841967 34.161618) (end 217.189759 30.50941) (width 0.25) (layer "B.Cu") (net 14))
 (segment (start 220.841967 35.38441) (end 220.841967 34.161618) (width 0.25) (layer "B.Cu") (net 14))
 (segment (start 210.466967 46.28441) (end 211.786967 44.96441) (width 0.4) (layer "F.Cu") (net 1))
 (segment (start 212.739967 45.91741) (end 211.786967 44.96441) (width 0.25) (layer "F.Cu") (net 1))
 (segment (start 208.291967 46.28441) (end 210.466967 46.28441) (width 0.4) (layer "F.Cu") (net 1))
 (segment (start 218.771967 45.91741) (end 212.739967 45.91741) (width 0.25) (layer "F.Cu") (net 1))
 (segment (start 217.891967 42.98441) (end 217.891967 45.03741) (width 0.25) (layer "B.Cu") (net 1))
 (segment (start 218.488124 45.91741) (end 218.771967 45.91741) (width 0.25) (layer "B.Cu") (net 1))
 (segment (start 217.891967 45.03741) (end 218.771967 45.91741) (width 0.25) (layer "B.Cu") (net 1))
 (segment (start 217.891967 46.513567) (end 218.488124 45.91741) (width 0.25) (layer "B.Cu") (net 1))
 (segment (start 217.891967 49.18441) (end 217.891967 46.513567) (width 0.25) (layer "B.Cu") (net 1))
 (segment (start 224.214466 39.54) (end 224.511967 39.837501) (width 0.4) (layer "B.Cu") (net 5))
 (segment (start 215.826967 43.013033) (end 219.3 39.54) (width 0.4) (layer "B.Cu") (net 5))
 (segment (start 215.826967 43.68441) (end 215.826967 43.013033) (width 0.4) (layer "B.Cu") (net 5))
 (segment (start 224.511967 39.837501) (end 224.511967 40.17641) (width 0.4) (layer "B.Cu") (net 5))
 (segment (start 215.676967 43.83441) (end 215.826967 43.68441) (width 0.4) (layer "B.Cu") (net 5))
 (segment (start 219.3 39.54) (end 224.214466 39.54) (width 0.4) (layer "B.Cu") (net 5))
 (segment (start 221.591967 49.18441) (end 221.92 48.856377) (width 0.25) (layer "B.Cu") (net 2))
 (segment (start 221.92 48.856377) (end 221.92 46.2416) (width 0.25) (layer "B.Cu") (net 2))
 (segment (start 221.591967 45.63741) (end 221.311967 45.91741) (width 0.25) (layer "B.Cu") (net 2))
 (segment (start 221.591967 42.98441) (end 221.591967 45.63741) (width 0.25) (layer "B.Cu") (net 2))
 (segment (start 221.92 46.2416) (end 221.59581 45.91741) (width 0.25) (layer "B.Cu") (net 2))
 (segment (start 221.59581 45.91741) (end 221.311967 45.91741) (width 0.25) (layer "B.Cu") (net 2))
 (segment (start 211.576967 48.28441) (end 208.291967 48.28441) (width 0.4) (layer "B.Cu") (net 19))
 (segment (start 214.526967 45.33441) (end 211.576967 48.28441) (width 0.4) (layer "B.Cu") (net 19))
 (segment (start 215.676967 45.33441) (end 214.526967 45.33441) (width 0.4) (layer "B.Cu") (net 19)))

